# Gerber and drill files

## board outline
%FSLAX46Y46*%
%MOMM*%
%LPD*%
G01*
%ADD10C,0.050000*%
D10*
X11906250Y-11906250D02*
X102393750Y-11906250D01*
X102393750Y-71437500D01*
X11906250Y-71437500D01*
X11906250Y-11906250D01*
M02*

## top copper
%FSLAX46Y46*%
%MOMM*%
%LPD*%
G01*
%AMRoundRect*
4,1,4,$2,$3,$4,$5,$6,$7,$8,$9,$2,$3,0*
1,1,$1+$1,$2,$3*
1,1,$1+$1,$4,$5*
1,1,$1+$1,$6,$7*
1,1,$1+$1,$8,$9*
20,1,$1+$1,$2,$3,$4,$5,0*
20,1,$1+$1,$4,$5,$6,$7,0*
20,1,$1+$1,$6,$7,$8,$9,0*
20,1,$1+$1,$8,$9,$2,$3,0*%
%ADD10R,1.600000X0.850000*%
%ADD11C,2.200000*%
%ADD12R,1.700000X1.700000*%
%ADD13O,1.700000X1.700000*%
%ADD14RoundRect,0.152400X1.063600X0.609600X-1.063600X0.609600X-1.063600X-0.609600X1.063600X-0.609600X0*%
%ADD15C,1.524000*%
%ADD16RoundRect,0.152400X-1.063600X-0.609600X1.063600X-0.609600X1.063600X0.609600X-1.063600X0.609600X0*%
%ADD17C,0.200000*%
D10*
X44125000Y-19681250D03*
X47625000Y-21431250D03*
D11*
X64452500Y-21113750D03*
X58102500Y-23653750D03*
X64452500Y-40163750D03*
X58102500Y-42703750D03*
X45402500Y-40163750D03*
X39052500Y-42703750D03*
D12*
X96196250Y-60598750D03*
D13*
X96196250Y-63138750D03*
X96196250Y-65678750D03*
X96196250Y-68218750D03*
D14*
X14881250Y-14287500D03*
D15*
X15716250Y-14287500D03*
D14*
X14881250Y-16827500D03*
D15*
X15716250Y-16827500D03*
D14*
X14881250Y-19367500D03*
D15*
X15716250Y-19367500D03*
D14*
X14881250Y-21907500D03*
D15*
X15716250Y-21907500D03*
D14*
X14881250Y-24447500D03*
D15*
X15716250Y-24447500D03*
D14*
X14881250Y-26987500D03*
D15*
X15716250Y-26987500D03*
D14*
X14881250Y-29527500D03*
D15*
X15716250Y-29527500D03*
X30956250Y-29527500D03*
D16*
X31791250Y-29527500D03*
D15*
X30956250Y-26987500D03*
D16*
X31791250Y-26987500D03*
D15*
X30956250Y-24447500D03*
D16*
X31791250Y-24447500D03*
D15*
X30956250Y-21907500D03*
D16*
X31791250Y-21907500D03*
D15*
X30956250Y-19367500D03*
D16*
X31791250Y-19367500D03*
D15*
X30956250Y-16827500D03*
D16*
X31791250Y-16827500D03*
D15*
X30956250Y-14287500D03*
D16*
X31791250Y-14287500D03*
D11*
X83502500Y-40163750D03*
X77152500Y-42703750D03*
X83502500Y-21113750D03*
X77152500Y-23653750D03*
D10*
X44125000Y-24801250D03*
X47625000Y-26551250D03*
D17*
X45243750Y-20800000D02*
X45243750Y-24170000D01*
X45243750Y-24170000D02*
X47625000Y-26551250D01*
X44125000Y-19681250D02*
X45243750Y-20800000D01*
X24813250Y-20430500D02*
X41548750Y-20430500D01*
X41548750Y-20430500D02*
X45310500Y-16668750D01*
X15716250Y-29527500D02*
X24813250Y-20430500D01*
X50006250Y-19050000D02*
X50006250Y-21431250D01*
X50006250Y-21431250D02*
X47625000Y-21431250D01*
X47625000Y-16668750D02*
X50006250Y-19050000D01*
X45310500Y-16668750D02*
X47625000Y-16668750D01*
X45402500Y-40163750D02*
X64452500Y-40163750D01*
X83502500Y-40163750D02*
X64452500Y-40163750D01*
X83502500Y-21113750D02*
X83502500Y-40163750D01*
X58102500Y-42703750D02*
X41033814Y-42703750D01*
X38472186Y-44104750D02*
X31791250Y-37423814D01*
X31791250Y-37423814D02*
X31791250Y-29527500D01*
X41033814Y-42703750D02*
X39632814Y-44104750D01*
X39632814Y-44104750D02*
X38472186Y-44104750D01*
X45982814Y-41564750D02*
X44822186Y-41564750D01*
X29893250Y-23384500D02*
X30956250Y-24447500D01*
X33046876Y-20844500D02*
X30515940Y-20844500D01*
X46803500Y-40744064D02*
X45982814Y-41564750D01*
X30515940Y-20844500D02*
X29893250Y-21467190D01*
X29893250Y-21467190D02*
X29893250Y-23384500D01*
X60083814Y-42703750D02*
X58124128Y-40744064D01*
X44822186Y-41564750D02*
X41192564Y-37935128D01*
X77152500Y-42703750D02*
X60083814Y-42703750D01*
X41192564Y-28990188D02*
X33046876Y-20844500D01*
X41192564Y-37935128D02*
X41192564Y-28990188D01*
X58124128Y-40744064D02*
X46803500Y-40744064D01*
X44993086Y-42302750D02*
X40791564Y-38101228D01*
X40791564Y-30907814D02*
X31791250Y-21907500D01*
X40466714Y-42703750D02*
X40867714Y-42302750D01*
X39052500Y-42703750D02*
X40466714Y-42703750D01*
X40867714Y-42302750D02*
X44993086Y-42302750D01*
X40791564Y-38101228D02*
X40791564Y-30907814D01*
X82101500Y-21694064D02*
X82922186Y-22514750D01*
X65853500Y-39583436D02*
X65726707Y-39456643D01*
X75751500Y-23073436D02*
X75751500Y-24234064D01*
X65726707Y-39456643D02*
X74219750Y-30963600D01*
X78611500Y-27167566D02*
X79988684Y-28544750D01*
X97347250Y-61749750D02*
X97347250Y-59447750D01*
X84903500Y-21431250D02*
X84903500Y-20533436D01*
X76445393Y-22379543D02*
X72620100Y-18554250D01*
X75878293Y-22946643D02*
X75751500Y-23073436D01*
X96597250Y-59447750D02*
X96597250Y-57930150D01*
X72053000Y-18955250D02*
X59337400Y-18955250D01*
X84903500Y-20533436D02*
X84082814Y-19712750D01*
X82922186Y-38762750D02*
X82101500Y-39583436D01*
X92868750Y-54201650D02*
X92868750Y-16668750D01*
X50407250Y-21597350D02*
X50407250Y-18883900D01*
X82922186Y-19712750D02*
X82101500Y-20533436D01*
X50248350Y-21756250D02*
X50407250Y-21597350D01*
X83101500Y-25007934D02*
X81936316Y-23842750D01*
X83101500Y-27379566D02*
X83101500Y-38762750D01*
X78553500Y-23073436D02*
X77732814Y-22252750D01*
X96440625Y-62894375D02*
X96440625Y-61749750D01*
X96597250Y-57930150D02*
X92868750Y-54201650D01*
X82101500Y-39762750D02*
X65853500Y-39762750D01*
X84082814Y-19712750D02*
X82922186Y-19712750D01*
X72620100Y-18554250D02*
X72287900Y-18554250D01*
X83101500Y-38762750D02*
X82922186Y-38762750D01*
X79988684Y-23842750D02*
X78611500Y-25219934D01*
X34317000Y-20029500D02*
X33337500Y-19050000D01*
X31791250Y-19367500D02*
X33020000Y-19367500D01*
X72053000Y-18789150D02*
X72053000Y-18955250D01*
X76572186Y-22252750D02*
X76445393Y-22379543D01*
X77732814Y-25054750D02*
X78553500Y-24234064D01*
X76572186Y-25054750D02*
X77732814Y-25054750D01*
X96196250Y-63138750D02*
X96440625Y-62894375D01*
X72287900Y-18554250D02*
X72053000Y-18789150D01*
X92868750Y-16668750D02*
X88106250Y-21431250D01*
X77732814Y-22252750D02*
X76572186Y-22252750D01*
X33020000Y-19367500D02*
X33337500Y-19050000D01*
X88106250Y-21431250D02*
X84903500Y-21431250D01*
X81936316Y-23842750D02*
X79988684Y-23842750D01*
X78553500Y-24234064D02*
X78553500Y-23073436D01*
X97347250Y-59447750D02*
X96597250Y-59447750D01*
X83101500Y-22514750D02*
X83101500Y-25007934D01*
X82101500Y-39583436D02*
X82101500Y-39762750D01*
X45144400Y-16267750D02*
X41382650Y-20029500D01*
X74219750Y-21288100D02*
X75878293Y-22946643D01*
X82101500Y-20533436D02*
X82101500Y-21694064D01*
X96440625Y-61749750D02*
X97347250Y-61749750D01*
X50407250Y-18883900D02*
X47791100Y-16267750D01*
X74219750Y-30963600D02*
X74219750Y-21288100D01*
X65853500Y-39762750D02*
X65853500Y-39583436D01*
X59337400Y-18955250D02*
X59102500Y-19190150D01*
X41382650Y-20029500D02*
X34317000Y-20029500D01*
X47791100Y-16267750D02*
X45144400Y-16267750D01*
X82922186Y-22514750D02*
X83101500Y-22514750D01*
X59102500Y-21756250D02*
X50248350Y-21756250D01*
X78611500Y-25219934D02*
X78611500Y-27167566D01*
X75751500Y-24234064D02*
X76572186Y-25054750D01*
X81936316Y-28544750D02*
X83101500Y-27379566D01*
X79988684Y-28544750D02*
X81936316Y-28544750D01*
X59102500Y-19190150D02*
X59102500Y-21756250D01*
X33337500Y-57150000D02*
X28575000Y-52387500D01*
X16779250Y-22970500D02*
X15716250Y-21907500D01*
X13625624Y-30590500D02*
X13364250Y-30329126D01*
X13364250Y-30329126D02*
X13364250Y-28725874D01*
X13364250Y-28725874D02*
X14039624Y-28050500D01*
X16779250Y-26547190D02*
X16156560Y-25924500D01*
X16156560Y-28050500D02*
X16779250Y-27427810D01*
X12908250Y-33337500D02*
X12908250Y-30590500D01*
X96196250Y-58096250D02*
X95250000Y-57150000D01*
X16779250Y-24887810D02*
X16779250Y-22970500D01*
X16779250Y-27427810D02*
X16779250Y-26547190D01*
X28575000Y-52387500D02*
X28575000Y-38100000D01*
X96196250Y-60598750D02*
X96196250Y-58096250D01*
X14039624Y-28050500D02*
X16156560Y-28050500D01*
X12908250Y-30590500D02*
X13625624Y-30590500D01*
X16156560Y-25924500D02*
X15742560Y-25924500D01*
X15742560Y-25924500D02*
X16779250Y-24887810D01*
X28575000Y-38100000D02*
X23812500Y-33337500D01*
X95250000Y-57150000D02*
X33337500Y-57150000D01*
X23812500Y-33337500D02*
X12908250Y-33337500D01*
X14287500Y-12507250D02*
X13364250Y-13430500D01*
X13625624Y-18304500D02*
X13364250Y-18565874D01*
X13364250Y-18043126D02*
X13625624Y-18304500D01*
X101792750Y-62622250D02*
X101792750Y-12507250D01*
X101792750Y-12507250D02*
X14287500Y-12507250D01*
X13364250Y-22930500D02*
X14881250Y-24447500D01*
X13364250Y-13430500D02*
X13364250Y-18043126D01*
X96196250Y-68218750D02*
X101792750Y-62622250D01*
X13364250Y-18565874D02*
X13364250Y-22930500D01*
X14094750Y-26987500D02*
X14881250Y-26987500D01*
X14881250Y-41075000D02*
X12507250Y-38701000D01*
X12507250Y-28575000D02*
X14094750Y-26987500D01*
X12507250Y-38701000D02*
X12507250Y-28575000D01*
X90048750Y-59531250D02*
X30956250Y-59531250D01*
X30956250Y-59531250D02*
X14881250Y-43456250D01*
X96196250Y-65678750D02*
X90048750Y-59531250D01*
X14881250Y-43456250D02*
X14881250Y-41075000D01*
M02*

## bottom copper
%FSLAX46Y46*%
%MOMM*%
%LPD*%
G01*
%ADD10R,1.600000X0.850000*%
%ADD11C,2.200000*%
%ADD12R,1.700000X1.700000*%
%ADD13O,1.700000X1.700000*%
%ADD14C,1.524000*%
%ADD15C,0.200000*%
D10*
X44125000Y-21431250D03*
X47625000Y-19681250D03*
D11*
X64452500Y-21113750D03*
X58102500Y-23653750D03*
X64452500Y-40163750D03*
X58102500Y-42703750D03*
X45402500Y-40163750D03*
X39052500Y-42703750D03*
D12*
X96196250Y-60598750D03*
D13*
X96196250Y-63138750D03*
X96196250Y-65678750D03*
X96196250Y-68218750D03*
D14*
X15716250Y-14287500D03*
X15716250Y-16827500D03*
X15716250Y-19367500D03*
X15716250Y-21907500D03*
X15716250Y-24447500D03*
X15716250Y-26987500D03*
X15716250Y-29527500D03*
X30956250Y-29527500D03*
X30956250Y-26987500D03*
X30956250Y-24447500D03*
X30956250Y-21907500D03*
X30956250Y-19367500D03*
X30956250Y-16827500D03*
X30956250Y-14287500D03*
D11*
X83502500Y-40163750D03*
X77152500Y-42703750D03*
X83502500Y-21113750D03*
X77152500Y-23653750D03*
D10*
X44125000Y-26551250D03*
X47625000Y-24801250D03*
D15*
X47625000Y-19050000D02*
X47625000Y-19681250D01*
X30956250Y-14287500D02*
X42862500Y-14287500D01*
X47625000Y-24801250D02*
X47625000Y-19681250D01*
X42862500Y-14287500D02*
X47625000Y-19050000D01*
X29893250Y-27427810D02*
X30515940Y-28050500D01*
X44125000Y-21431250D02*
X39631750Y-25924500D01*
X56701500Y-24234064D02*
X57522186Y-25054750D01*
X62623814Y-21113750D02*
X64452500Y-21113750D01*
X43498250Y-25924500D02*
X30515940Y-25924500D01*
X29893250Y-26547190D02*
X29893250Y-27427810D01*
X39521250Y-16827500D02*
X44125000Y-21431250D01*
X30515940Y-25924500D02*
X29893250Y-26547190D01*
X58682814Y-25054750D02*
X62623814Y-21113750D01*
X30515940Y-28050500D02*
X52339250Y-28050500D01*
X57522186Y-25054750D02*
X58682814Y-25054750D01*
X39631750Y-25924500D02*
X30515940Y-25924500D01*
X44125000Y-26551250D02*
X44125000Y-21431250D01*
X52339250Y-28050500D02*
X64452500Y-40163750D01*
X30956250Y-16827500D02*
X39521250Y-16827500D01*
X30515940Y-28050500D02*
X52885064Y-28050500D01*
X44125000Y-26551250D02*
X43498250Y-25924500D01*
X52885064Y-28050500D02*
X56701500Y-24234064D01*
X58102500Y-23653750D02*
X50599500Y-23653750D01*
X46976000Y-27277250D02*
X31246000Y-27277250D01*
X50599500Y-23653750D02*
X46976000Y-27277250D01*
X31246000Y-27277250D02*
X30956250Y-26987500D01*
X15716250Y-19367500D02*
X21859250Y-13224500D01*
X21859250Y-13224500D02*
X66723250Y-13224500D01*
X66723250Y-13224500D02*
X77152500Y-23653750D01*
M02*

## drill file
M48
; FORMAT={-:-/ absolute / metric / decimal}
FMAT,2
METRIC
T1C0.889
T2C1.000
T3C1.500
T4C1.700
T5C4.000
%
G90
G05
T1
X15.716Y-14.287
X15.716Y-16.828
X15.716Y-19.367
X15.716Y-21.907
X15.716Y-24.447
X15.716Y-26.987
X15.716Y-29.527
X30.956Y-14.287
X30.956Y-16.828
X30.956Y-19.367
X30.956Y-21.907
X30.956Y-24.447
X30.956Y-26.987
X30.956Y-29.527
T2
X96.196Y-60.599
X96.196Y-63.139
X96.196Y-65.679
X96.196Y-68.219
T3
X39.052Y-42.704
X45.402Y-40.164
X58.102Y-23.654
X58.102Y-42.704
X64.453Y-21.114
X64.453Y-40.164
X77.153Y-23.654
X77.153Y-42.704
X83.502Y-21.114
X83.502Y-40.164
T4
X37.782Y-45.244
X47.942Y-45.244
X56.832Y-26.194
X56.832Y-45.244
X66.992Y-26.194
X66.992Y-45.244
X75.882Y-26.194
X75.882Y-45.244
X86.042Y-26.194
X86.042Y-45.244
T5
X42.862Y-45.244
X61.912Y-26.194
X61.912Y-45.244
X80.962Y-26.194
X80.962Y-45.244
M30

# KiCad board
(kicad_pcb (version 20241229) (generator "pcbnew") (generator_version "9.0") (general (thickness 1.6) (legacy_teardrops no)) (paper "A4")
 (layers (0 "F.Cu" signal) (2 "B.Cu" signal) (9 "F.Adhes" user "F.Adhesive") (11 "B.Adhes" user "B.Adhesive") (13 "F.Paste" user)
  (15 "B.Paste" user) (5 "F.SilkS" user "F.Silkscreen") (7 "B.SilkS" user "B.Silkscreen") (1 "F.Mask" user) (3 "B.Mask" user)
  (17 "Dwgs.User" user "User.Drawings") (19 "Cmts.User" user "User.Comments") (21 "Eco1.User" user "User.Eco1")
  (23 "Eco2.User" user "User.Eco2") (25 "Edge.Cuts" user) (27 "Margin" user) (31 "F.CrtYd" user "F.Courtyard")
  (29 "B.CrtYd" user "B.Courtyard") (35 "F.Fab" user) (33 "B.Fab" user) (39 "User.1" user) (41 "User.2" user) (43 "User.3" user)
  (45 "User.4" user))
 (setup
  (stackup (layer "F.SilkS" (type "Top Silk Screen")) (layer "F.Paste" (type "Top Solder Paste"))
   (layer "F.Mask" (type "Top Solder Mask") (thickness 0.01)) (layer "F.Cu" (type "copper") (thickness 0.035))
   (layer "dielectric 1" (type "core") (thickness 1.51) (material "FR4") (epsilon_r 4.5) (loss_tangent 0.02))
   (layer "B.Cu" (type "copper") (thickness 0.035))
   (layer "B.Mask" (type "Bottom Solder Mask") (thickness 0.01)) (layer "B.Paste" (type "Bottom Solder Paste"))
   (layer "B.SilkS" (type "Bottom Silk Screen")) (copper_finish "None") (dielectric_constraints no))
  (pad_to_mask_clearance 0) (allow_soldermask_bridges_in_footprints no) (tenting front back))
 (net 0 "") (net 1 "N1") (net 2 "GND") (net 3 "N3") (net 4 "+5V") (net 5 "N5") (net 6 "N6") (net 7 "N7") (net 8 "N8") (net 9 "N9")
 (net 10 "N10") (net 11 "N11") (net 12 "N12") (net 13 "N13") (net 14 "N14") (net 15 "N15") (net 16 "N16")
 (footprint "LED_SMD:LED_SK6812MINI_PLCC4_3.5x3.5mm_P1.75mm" (layer "F.Cu") (at 45.875 20.55625)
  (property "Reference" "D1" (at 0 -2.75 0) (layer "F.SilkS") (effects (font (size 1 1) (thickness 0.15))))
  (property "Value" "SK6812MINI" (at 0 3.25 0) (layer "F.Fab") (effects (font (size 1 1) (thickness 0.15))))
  (pad "1" smd rect (at -1.75 -0.875) (size 1.6 0.85) (layers "F.Cu" "F.Mask" "F.Paste") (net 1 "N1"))
  (pad "2" smd rect (at -1.75 0.875) (size 1.6 0.85) (layers "F.Mask" "B.Cu" "F.Paste") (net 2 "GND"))
  (pad "3" smd rect (at 1.75 0.875) (size 1.6 0.85) (layers "F.Cu" "F.Mask" "F.Paste") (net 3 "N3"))
  (pad "4" smd rect (at 1.75 -0.875) (size 1.6 0.85) (layers "F.Mask" "B.Cu" "F.Paste") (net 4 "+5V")))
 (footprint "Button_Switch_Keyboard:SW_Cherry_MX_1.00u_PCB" (layer "F.Cu") (at 64.4525 21.11375)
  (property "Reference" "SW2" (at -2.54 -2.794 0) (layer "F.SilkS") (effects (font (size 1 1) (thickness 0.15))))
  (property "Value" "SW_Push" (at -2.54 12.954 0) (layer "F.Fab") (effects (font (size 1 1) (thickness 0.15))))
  (pad "" np_thru_hole circle (at -7.62 5.08) (size 1.7 1.7) (drill 1.7) (layers "*.Cu" "*.Mask"))
  (pad "" np_thru_hole circle (at -2.54 5.08) (size 4 4) (drill 4) (layers "*.Cu" "*.Mask"))
  (pad "" np_thru_hole circle (at 2.54 5.08) (size 1.7 1.7) (drill 1.7) (layers "*.Cu" "*.Mask"))
  (pad "1" thru_hole circle (at 0 0) (size 2.2 2.2) (drill 1.5) (layers "*.Cu" "*.Mask") (remove_unused_layers no) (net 2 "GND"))
  (pad "2" thru_hole circle (at -6.35 2.54) (size 2.2 2.2) (drill 1.5) (layers "*.Cu" "*.Mask") (remove_unused_layers no) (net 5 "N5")))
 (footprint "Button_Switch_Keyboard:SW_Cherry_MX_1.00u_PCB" (layer "F.Cu") (at 64.4525 40.16375)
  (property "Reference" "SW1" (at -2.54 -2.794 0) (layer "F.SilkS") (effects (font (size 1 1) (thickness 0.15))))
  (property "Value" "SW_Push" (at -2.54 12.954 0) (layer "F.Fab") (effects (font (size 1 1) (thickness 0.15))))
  (pad "" np_thru_hole circle (at -7.62 5.08) (size 1.7 1.7) (drill 1.7) (layers "*.Cu" "*.Mask"))
  (pad "" np_thru_hole circle (at -2.54 5.08) (size 4 4) (drill 4) (layers "*.Cu" "*.Mask"))
  (pad "" np_thru_hole circle (at 2.54 5.08) (size 1.7 1.7) (drill 1.7) (layers "*.Cu" "*.Mask"))
  (pad "1" thru_hole circle (at 0 0) (size 2.2 2.2) (drill 1.5) (layers "*.Cu" "*.Mask") (remove_unused_layers no) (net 2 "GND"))
  (pad "2" thru_hole circle (at -6.35 2.54) (size 2.2 2.2) (drill 1.5) (layers "*.Cu" "*.Mask") (remove_unused_layers no) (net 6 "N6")))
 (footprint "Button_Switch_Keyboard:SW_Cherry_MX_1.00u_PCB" (layer "F.Cu") (at 45.4025 40.16375)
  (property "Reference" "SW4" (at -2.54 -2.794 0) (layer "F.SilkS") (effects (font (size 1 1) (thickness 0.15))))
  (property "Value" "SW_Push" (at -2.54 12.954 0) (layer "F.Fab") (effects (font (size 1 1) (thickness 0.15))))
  (pad "" np_thru_hole circle (at -7.62 5.08) (size 1.7 1.7) (drill 1.7) (layers "*.Cu" "*.Mask"))
  (pad "" np_thru_hole circle (at -2.54 5.08) (size 4 4) (drill 4) (layers "*.Cu" "*.Mask"))
  (pad "" np_thru_hole circle (at 2.54 5.08) (size 1.7 1.7) (drill 1.7) (layers "*.Cu" "*.Mask"))
  (pad "1" thru_hole circle (at 0 0) (size 2.2 2.2) (drill 1.5) (layers "*.Cu" "*.Mask") (remove_unused_layers no) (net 2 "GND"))
  (pad "2" thru_hole circle (at -6.35 2.54) (size 2.2 2.2) (drill 1.5) (layers "*.Cu" "*.Mask") (remove_unused_layers no) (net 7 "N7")))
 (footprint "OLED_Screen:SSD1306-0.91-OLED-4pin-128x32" (layer "F.Cu") (at 59.69625 58.40875)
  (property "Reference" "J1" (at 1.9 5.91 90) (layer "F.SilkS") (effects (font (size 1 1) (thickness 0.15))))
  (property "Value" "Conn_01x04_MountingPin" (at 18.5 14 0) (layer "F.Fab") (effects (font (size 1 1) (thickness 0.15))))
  (pad "1" thru_hole rect (at 36.5 2.19) (size 1.7 1.7) (drill 1) (layers "*.Cu" "*.Mask") (remove_unused_layers no) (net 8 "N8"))
  (pad "2" thru_hole oval (at 36.5 4.73) (size 1.7 1.7) (drill 1) (layers "*.Cu" "*.Mask") (remove_unused_layers no) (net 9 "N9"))
  (pad "3" thru_hole oval (at 36.5 7.27) (size 1.7 1.7) (drill 1) (layers "*.Cu" "*.Mask") (remove_unused_layers no) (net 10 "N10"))
  (pad "4" thru_hole oval (at 36.5 9.81) (size 1.7 1.7) (drill 1) (layers "*.Cu" "*.Mask") (remove_unused_layers no) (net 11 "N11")))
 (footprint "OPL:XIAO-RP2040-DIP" (layer "F.Cu") (at 23.33625 21.9075)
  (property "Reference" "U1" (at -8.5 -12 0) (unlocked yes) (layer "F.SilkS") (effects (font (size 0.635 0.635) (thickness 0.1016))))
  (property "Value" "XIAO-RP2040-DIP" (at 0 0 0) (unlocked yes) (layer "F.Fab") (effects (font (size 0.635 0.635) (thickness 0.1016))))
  (pad "1" smd roundrect (at -8.455 -7.62 180) (size 2.432 1.524) (layers "F.Cu" "F.Mask") (roundrect_rratio 0.1) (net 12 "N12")
   (thermal_bridge_angle 45))
  (pad "1" thru_hole circle (at -7.62 -7.62 180) (size 1.524 1.524) (drill 0.889) (layers "*.Cu" "*.Mask") (remove_unused_layers no)
   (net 12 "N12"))
  (pad "2" smd roundrect (at -8.455 -5.08 180) (size 2.432 1.524) (layers "F.Cu" "F.Mask") (roundrect_rratio 0.1) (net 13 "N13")
   (thermal_bridge_angle 45))
  (pad "2" thru_hole circle (at -7.62 -5.08 180) (size 1.524 1.524) (drill 0.889) (layers "*.Cu" "*.Mask") (remove_unused_layers no)
   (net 13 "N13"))
  (pad "3" smd roundrect (at -8.455 -2.54 180) (size 2.432 1.524) (layers "F.Cu" "F.Mask") (roundrect_rratio 0.1) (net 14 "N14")
   (thermal_bridge_angle 45))
  (pad "3" thru_hole circle (at -7.62 -2.54 180) (size 1.524 1.524) (drill 0.889) (layers "*.Cu" "*.Mask") (remove_unused_layers no)
   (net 14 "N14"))
  (pad "4" smd roundrect (at -8.455 0 180) (size 2.432 1.524) (layers "F.Cu" "F.Mask") (roundrect_rratio 0.1) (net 8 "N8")
   (thermal_bridge_angle 45))
  (pad "4" thru_hole circle (at -7.62 0 180) (size 1.524 1.524) (drill 0.889) (layers "*.Cu" "*.Mask") (remove_unused_layers no)
   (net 8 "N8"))
  (pad "5" smd roundrect (at -8.455 2.54 180) (size 2.432 1.524) (layers "F.Cu" "F.Mask") (roundrect_rratio 0.1) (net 11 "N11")
   (thermal_bridge_angle 45))
  (pad "5" thru_hole circle (at -7.62 2.54 180) (size 1.524 1.524) (drill 0.889) (layers "*.Cu" "*.Mask") (remove_unused_layers no)
   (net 11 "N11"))
  (pad "6" smd roundrect (at -8.455 5.08 180) (size 2.432 1.524) (layers "F.Cu" "F.Mask") (roundrect_rratio 0.1) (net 10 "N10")
   (thermal_bridge_angle 45))
  (pad "6" thru_hole circle (at -7.62 5.08 180) (size 1.524 1.524) (drill 0.889) (layers "*.Cu" "*.Mask") (remove_unused_layers no)
   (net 10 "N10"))
  (pad "7" smd roundrect (at -8.455 7.62 180) (size 2.432 1.524) (layers "F.Cu" "F.Mask") (roundrect_rratio 0.1) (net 3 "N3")
   (thermal_bridge_angle 45))
  (pad "7" thru_hole circle (at -7.62 7.62 180) (size 1.524 1.524) (drill 0.889) (layers "*.Cu" "*.Mask") (remove_unused_layers no)
   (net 3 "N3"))
  (pad "8" thru_hole circle (at 7.62 7.62) (size 1.524 1.524) (drill 0.889) (layers "*.Cu" "*.Mask") (remove_unused_layers no) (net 6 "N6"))
  (pad "8" smd roundrect (at 8.455 7.62) (size 2.432 1.524) (layers "F.Cu" "F.Mask") (roundrect_rratio 0.1) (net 6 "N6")
   (thermal_bridge_angle 45))
  (pad "9" thru_hole circle (at 7.62 5.08) (size 1.524 1.524) (drill 0.889) (layers "*.Cu" "*.Mask") (remove_unused_layers no) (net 5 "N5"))
  (pad "9" smd roundrect (at 8.455 5.08) (size 2.432 1.524) (layers "F.Cu" "F.Mask") (roundrect_rratio 0.1) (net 5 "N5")
   (thermal_bridge_angle 45))
  (pad "10" thru_hole circle (at 7.62 2.54) (size 1.524 1.524) (drill 0.889) (layers "*.Cu" "*.Mask") (remove_unused_layers no)
   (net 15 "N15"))
  (pad "10" smd roundrect (at 8.455 2.54) (size 2.432 1.524) (layers "F.Cu" "F.Mask") (roundrect_rratio 0.1) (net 15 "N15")
   (thermal_bridge_angle 45))
  (pad "11" thru_hole circle (at 7.62 0) (size 1.524 1.524) (drill 0.889) (layers "*.Cu" "*.Mask") (remove_unused_layers no) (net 7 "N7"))
  (pad "11" smd roundrect (at 8.455 0) (size 2.432 1.524) (layers "F.Cu" "F.Mask") (roundrect_rratio 0.1) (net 7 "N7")
   (thermal_bridge_angle 45))
  (pad "12" thru_hole circle (at 7.62 -2.54) (size 1.524 1.524) (drill 0.889) (layers "*.Cu" "*.Mask") (remove_unused_layers no)
   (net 9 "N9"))
  (pad "12" smd roundrect (at 8.455 -2.54) (size 2.432 1.524) (layers "F.Cu" "F.Mask") (roundrect_rratio 0.1) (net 9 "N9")
   (thermal_bridge_angle 45))
  (pad "13" thru_hole circle (at 7.62 -5.08) (size 1.524 1.524) (drill 0.889) (layers "*.Cu" "*.Mask") (remove_unused_layers no)
   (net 2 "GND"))
  (pad "13" smd roundrect (at 8.455 -5.08) (size 2.432 1.524) (layers "F.Cu" "F.Mask") (roundrect_rratio 0.1) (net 2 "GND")
   (thermal_bridge_angle 45))
  (pad "14" thru_hole circle (at 7.62 -7.62) (size 1.524 1.524) (drill 0.889) (layers "*.Cu" "*.Mask") (remove_unused_layers no)
   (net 4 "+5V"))
  (pad "14" smd roundrect (at 8.455 -7.62) (size 2.432 1.524) (layers "F.Cu" "F.Mask") (roundrect_rratio 0.1) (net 4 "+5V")
   (thermal_bridge_angle 45)))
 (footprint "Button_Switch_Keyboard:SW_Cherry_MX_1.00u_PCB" (layer "F.Cu") (at 83.5025 40.16375)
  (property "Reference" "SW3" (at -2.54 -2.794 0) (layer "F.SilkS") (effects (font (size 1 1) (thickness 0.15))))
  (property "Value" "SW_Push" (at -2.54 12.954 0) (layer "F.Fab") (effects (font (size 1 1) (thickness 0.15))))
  (pad "" np_thru_hole circle (at -7.62 5.08) (size 1.7 1.7) (drill 1.7) (layers "*.Cu" "*.Mask"))
  (pad "" np_thru_hole circle (at -2.54 5.08) (size 4 4) (drill 4) (layers "*.Cu" "*.Mask"))
  (pad "" np_thru_hole circle (at 2.54 5.08) (size 1.7 1.7) (drill 1.7) (layers "*.Cu" "*.Mask"))
  (pad "1" thru_hole circle (at 0 0) (size 2.2 2.2) (drill 1.5) (layers "*.Cu" "*.Mask") (remove_unused_layers no) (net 2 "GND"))
  (pad "2" thru_hole circle (at -6.35 2.54) (size 2.2 2.2) (drill 1.5) (layers "*.Cu" "*.Mask") (remove_unused_layers no) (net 15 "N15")))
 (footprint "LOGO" (layer "F.Cu") (at 21.43125 61.9125)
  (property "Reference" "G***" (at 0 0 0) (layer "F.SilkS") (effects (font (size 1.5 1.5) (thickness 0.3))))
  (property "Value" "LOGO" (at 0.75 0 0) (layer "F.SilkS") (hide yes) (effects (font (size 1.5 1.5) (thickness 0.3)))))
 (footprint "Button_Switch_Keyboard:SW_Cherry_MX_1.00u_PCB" (layer "F.Cu") (at 83.5025 21.11375)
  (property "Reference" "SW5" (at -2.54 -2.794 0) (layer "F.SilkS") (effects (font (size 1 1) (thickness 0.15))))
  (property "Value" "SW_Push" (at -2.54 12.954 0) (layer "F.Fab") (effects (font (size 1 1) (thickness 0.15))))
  (pad "" np_thru_hole circle (at -7.62 5.08) (size 1.7 1.7) (drill 1.7) (layers "*.Cu" "*.Mask"))
  (pad "" np_thru_hole circle (at -2.54 5.08) (size 4 4) (drill 4) (layers "*.Cu" "*.Mask"))
  (pad "" np_thru_hole circle (at 2.54 5.08) (size 1.7 1.7) (drill 1.7) (layers "*.Cu" "*.Mask"))
  (pad "1" thru_hole circle (at 0 0) (size 2.2 2.2) (drill 1.5) (layers "*.Cu" "*.Mask") (remove_unused_layers no) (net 2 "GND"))
  (pad "2" thru_hole circle (at -6.35 2.54) (size 2.2 2.2) (drill 1.5) (layers "*.Cu" "*.Mask") (remove_unused_layers no) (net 14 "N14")))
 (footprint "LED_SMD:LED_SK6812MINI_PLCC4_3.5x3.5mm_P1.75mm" (layer "F.Cu") (at 45.875 25.67625)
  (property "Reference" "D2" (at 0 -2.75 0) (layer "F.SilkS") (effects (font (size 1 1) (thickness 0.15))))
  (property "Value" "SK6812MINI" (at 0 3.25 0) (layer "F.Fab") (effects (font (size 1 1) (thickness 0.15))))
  (pad "1" smd rect (at -1.75 -0.875) (size 1.6 0.85) (layers "F.Cu" "F.Mask" "F.Paste") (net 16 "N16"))
  (pad "2" smd rect (at -1.75 0.875) (size 1.6 0.85) (layers "F.Mask" "B.Cu" "F.Paste") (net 2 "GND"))
  (pad "3" smd rect (at 1.75 0.875) (size 1.6 0.85) (layers "F.Cu" "F.Mask" "F.Paste") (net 1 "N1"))
  (pad "4" smd rect (at 1.75 -0.875) (size 1.6 0.85) (layers "F.Mask" "B.Cu" "F.Paste") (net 4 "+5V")))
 (gr_rect (start 11.90625 11.90625) (end 102.39375 71.4375) (stroke (width 0.05) (type default)) (fill no) (layer "Edge.Cuts"))
 (segment (start 45.24375 20.8) (end 45.24375 24.17) (width 0.2) (layer "F.Cu") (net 1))
 (segment (start 45.24375 24.17) (end 47.625 26.55125) (width 0.2) (layer "F.Cu") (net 1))
 (segment (start 44.125 19.68125) (end 45.24375 20.8) (width 0.2) (layer "F.Cu") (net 1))
 (segment (start 47.625 19.05) (end 47.625 19.68125) (width 0.2) (layer "B.Cu") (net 4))
 (segment (start 30.95625 14.2875) (end 42.8625 14.2875) (width 0.2) (layer "B.Cu") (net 4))
 (segment (start 47.625 24.80125) (end 47.625 19.68125) (width 0.2) (layer "B.Cu") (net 4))
 (segment (start 42.8625 14.2875) (end 47.625 19.05) (width 0.2) (layer "B.Cu") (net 4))
 (segment (start 24.81325 20.4305) (end 41.54875 20.4305) (width 0.2) (layer "F.Cu") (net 3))
 (segment (start 41.54875 20.4305) (end 45.3105 16.66875) (width 0.2) (layer "F.Cu") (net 3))
 (segment (start 15.71625 29.5275) (end 24.81325 20.4305) (width 0.2) (layer "F.Cu") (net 3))
 (segment (start 50.00625 19.05) (end 50.00625 21.43125) (width 0.2) (layer "F.Cu") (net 3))
 (segment (start 50.00625 21.43125) (end 47.625 21.43125) (width 0.2) (layer "F.Cu") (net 3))
 (segment (start 47.625 16.66875) (end 50.00625 19.05) (width 0.2) (layer "F.Cu") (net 3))
 (segment (start 45.3105 16.66875) (end 47.625 16.66875) (width 0.2) (layer "F.Cu") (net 3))
 (segment (start 45.4025 40.16375) (end 64.4525 40.16375) (width 0.2) (layer "F.Cu") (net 2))
 (segment (start 83.5025 40.16375) (end 64.4525 40.16375) (width 0.2) (layer "F.Cu") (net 2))
 (segment (start 83.5025 21.11375) (end 83.5025 40.16375) (width 0.2) (layer "F.Cu") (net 2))
 (segment (start 29.89325 27.42781) (end 30.51594 28.0505) (width 0.2) (layer "B.Cu") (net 2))
 (segment (start 44.125 21.43125) (end 39.63175 25.9245) (width 0.2) (layer "B.Cu") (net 2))
 (segment (start 56.7015 24.234064) (end 57.522186 25.05475) (width 0.2) (layer "B.Cu") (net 2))
 (segment (start 62.623814 21.11375) (end 64.4525 21.11375) (width 0.2) (layer "B.Cu") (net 2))
 (segment (start 43.49825 25.9245) (end 30.51594 25.9245) (width 0.2) (layer "B.Cu") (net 2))
 (segment (start 29.89325 26.54719) (end 29.89325 27.42781) (width 0.2) (layer "B.Cu") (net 2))
 (segment (start 39.52125 16.8275) (end 44.125 21.43125) (width 0.2) (layer "B.Cu") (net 2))
 (segment (start 30.51594 25.9245) (end 29.89325 26.54719) (width 0.2) (layer "B.Cu") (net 2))
 (segment (start 58.682814 25.05475) (end 62.623814 21.11375) (width 0.2) (layer "B.Cu") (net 2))
 (segment (start 30.51594 28.0505) (end 52.33925 28.0505) (width 0.2) (layer "B.Cu") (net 2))
 (segment (start 57.522186 25.05475) (end 58.682814 25.05475) (width 0.2) (layer "B.Cu") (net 2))
 (segment (start 39.63175 25.9245) (end 30.51594 25.9245) (width 0.2) (layer "B.Cu") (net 2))
 (segment (start 44.125 26.55125) (end 44.125 21.43125) (width 0.2) (layer "B.Cu") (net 2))
 (segment (start 52.33925 28.0505) (end 64.4525 40.16375) (width 0.2) (layer "B.Cu") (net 2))
 (segment (start 30.95625 16.8275) (end 39.52125 16.8275) (width 0.2) (layer "B.Cu") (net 2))
 (segment (start 30.51594 28.0505) (end 52.885064 28.0505) (width 0.2) (layer "B.Cu") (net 2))
 (segment (start 44.125 26.55125) (end 43.49825 25.9245) (width 0.2) (layer "B.Cu") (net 2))
 (segment (start 52.885064 28.0505) (end 56.7015 24.234064) (width 0.2) (layer "B.Cu") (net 2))
 (segment (start 58.1025 42.70375) (end 41.033814 42.70375) (width 0.2) (layer "F.Cu") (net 6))
 (segment (start 38.472186 44.10475) (end 31.79125 37.423814) (width 0.2) (layer "F.Cu") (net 6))
 (segment (start 31.79125 37.423814) (end 31.79125 29.5275) (width 0.2) (layer "F.Cu") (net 6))
 (segment (start 41.033814 42.70375) (end 39.632814 44.10475) (width 0.2) (layer "F.Cu") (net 6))
 (segment (start 39.632814 44.10475) (end 38.472186 44.10475) (width 0.2) (layer "F.Cu") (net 6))
 (segment (start 58.1025 23.65375) (end 50.5995 23.65375) (width 0.2) (layer "B.Cu") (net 5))
 (segment (start 46.976 27.27725) (end 31.246 27.27725) (width 0.2) (layer "B.Cu") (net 5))
 (segment (start 50.5995 23.65375) (end 46.976 27.27725) (width 0.2) (layer "B.Cu") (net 5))
 (segment (start 31.246 27.27725) (end 30.95625 26.9875) (width 0.2) (layer "B.Cu") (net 5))
 (segment (start 45.982814 41.56475) (end 44.822186 41.56475) (width 0.2) (layer "F.Cu") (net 15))
 (segment (start 29.89325 23.3845) (end 30.95625 24.4475) (width 0.2) (layer "F.Cu") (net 15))
 (segment (start 33.046876 20.8445) (end 30.51594 20.8445) (width 0.2) (layer "F.Cu") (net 15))
 (segment (start 46.8035 40.744064) (end 45.982814 41.56475) (width 0.2) (layer "F.Cu") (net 15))
 (segment (start 30.51594 20.8445) (end 29.89325 21.46719) (width 0.2) (layer "F.Cu") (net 15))
 (segment (start 29.89325 21.46719) (end 29.89325 23.3845) (width 0.2) (layer "F.Cu") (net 15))
 (segment (start 60.083814 42.70375) (end 58.124128 40.744064) (width 0.2) (layer "F.Cu") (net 15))
 (segment (start 44.822186 41.56475) (end 41.192564 37.935128) (width 0.2) (layer "F.Cu") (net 15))
 (segment (start 77.1525 42.70375) (end 60.083814 42.70375) (width 0.2) (layer "F.Cu") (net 15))
 (segment (start 41.192564 28.990188) (end 33.046876 20.8445) (width 0.2) (layer "F.Cu") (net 15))
 (segment (start 41.192564 37.935128) (end 41.192564 28.990188) (width 0.2) (layer "F.Cu") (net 15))
 (segment (start 58.124128 40.744064) (end 46.8035 40.744064) (width 0.2) (layer "F.Cu") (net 15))
 (segment (start 44.993086 42.30275) (end 40.791564 38.101228) (width 0.2) (layer "F.Cu") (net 7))
 (segment (start 40.791564 30.907814) (end 31.79125 21.9075) (width 0.2) (layer "F.Cu") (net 7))
 (segment (start 40.466714 42.70375) (end 40.867714 42.30275) (width 0.2) (layer "F.Cu") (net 7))
 (segment (start 39.0525 42.70375) (end 40.466714 42.70375) (width 0.2) (layer "F.Cu") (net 7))
 (segment (start 40.867714 42.30275) (end 44.993086 42.30275) (width 0.2) (layer "F.Cu") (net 7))
 (segment (start 40.791564 38.101228) (end 40.791564 30.907814) (width 0.2) (layer "F.Cu") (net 7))
 (segment (start 82.1015 21.694064) (end 82.922186 22.51475) (width 0.2) (layer "F.Cu") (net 9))
 (segment (start 65.8535 39.583436) (end 65.726707 39.456643) (width 0.2) (layer "F.Cu") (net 9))
 (segment (start 75.7515 23.073436) (end 75.7515 24.234064) (width 0.2) (layer "F.Cu") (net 9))
 (segment (start 65.726707 39.456643) (end 74.21975 30.9636) (width 0.2) (layer "F.Cu") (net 9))
 (segment (start 78.6115 27.167566) (end 79.988684 28.54475) (width 0.2) (layer "F.Cu") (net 9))
 (segment (start 97.34725 61.74975) (end 97.34725 59.44775) (width 0.2) (layer "F.Cu") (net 9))
 (segment (start 84.9035 21.43125) (end 84.9035 20.533436) (width 0.2) (layer "F.Cu") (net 9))
 (segment (start 76.445393 22.379543) (end 72.6201 18.55425) (width 0.2) (layer "F.Cu") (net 9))
 (segment (start 75.878293 22.946643) (end 75.7515 23.073436) (width 0.2) (layer "F.Cu") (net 9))
 (segment (start 96.59725 59.44775) (end 96.59725 57.93015) (width 0.2) (layer "F.Cu") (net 9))
 (segment (start 72.053 18.95525) (end 59.3374 18.95525) (width 0.2) (layer "F.Cu") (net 9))
 (segment (start 84.9035 20.533436) (end 84.082814 19.71275) (width 0.2) (layer "F.Cu") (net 9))
 (segment (start 82.922186 38.76275) (end 82.1015 39.583436) (width 0.2) (layer "F.Cu") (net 9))
 (segment (start 92.86875 54.20165) (end 92.86875 16.66875) (width 0.2) (layer "F.Cu") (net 9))
 (segment (start 50.40725 21.59735) (end 50.40725 18.8839) (width 0.2) (layer "F.Cu") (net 9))
 (segment (start 82.922186 19.71275) (end 82.1015 20.533436) (width 0.2) (layer "F.Cu") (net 9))
 (segment (start 50.24835 21.75625) (end 50.40725 21.59735) (width 0.2) (layer "F.Cu") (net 9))
 (segment (start 83.1015 25.007934) (end 81.936316 23.84275) (width 0.2) (layer "F.Cu") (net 9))
 (segment (start 83.1015 27.379566) (end 83.1015 38.76275) (width 0.2) (layer "F.Cu") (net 9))
 (segment (start 78.5535 23.073436) (end 77.732814 22.25275) (width 0.2) (layer "F.Cu") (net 9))
 (segment (start 96.440625 62.894375) (end 96.440625 61.74975) (width 0.2) (layer "F.Cu") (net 9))
 (segment (start 96.59725 57.93015) (end 92.86875 54.20165) (width 0.2) (layer "F.Cu") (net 9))
 (segment (start 82.1015 39.76275) (end 65.8535 39.76275) (width 0.2) (layer "F.Cu") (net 9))
 (segment (start 84.082814 19.71275) (end 82.922186 19.71275) (width 0.2) (layer "F.Cu") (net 9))
 (segment (start 72.6201 18.55425) (end 72.2879 18.55425) (width 0.2) (layer "F.Cu") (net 9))
 (segment (start 83.1015 38.76275) (end 82.922186 38.76275) (width 0.2) (layer "F.Cu") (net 9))
 (segment (start 79.988684 23.84275) (end 78.6115 25.219934) (width 0.2) (layer "F.Cu") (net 9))
 (segment (start 34.317 20.0295) (end 33.3375 19.05) (width 0.2) (layer "F.Cu") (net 9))
 (segment (start 31.79125 19.3675) (end 33.02 19.3675) (width 0.2) (layer "F.Cu") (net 9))
 (segment (start 72.053 18.78915) (end 72.053 18.95525) (width 0.2) (layer "F.Cu") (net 9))
 (segment (start 76.572186 22.25275) (end 76.445393 22.379543) (width 0.2) (layer "F.Cu") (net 9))
 (segment (start 77.732814 25.05475) (end 78.5535 24.234064) (width 0.2) (layer "F.Cu") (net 9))
 (segment (start 76.572186 25.05475) (end 77.732814 25.05475) (width 0.2) (layer "F.Cu") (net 9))
 (segment (start 96.19625 63.13875) (end 96.440625 62.894375) (width 0.2) (layer "F.Cu") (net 9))
 (segment (start 72.2879 18.55425) (end 72.053 18.78915) (width 0.2) (layer "F.Cu") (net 9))
 (segment (start 92.86875 16.66875) (end 88.10625 21.43125) (width 0.2) (layer "F.Cu") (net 9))
 (segment (start 77.732814 22.25275) (end 76.572186 22.25275) (width 0.2) (layer "F.Cu") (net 9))
 (segment (start 33.02 19.3675) (end 33.3375 19.05) (width 0.2) (layer "F.Cu") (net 9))
 (segment (start 88.10625 21.43125) (end 84.9035 21.43125) (width 0.2) (layer "F.Cu") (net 9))
 (segment (start 81.936316 23.84275) (end 79.988684 23.84275) (width 0.2) (layer "F.Cu") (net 9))
 (segment (start 78.5535 24.234064) (end 78.5535 23.073436) (width 0.2) (layer "F.Cu") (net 9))
 (segment (start 97.34725 59.44775) (end 96.59725 59.44775) (width 0.2) (layer "F.Cu") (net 9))
 (segment (start 83.1015 22.51475) (end 83.1015 25.007934) (width 0.2) (layer "F.Cu") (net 9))
 (segment (start 82.1015 39.583436) (end 82.1015 39.76275) (width 0.2) (layer "F.Cu") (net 9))
 (segment (start 45.1444 16.26775) (end 41.38265 20.0295) (width 0.2) (layer "F.Cu") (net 9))
 (segment (start 74.21975 21.2881) (end 75.878293 22.946643) (width 0.2) (layer "F.Cu") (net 9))
 (segment (start 82.1015 20.533436) (end 82.1015 21.694064) (width 0.2) (layer "F.Cu") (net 9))
 (segment (start 96.440625 61.74975) (end 97.34725 61.74975) (width 0.2) (layer "F.Cu") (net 9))
 (segment (start 50.40725 18.8839) (end 47.7911 16.26775) (width 0.2) (layer "F.Cu") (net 9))
 (segment (start 74.21975 30.9636) (end 74.21975 21.2881) (width 0.2) (layer "F.Cu") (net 9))
 (segment (start 65.8535 39.76275) (end 65.8535 39.583436) (width 0.2) (layer "F.Cu") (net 9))
 (segment (start 59.3374 18.95525) (end 59.1025 19.19015) (width 0.2) (layer "F.Cu") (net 9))
 (segment (start 41.38265 20.0295) (end 34.317 20.0295) (width 0.2) (layer "F.Cu") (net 9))
 (segment (start 47.7911 16.26775) (end 45.1444 16.26775) (width 0.2) (layer "F.Cu") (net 9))
 (segment (start 82.922186 22.51475) (end 83.1015 22.51475) (width 0.2) (layer "F.Cu") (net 9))
 (segment (start 59.1025 21.75625) (end 50.24835 21.75625) (width 0.2) (layer "F.Cu") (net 9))
 (segment (start 78.6115 25.219934) (end 78.6115 27.167566) (width 0.2) (layer "F.Cu") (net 9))
 (segment (start 75.7515 24.234064) (end 76.572186 25.05475) (width 0.2) (layer "F.Cu") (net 9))
 (segment (start 81.936316 28.54475) (end 83.1015 27.379566) (width 0.2) (layer "F.Cu") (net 9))
 (segment (start 79.988684 28.54475) (end 81.936316 28.54475) (width 0.2) (layer "F.Cu") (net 9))
 (segment (start 59.1025 19.19015) (end 59.1025 21.75625) (width 0.2) (layer "F.Cu") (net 9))
 (segment (start 33.3375 57.15) (end 28.575 52.3875) (width 0.2) (layer "F.Cu") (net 8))
 (segment (start 16.77925 22.9705) (end 15.71625 21.9075) (width 0.2) (layer "F.Cu") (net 8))
 (segment (start 13.625624 30.5905) (end 13.36425 30.329126) (width 0.2) (layer "F.Cu") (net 8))
 (segment (start 13.36425 30.329126) (end 13.36425 28.725874) (width 0.2) (layer "F.Cu") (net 8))
 (segment (start 13.36425 28.725874) (end 14.039624 28.0505) (width 0.2) (layer "F.Cu") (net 8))
 (segment (start 16.77925 26.54719) (end 16.15656 25.9245) (width 0.2) (layer "F.Cu") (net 8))
 (segment (start 16.15656 28.0505) (end 16.77925 27.42781) (width 0.2) (layer "F.Cu") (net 8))
 (segment (start 12.90825 33.3375) (end 12.90825 30.5905) (width 0.2) (layer "F.Cu") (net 8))
 (segment (start 96.19625 58.09625) (end 95.25 57.15) (width 0.2) (layer "F.Cu") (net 8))
 (segment (start 16.77925 24.88781) (end 16.77925 22.9705) (width 0.2) (layer "F.Cu") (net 8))
 (segment (start 16.77925 27.42781) (end 16.77925 26.54719) (width 0.2) (layer "F.Cu") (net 8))
 (segment (start 28.575 52.3875) (end 28.575 38.1) (width 0.2) (layer "F.Cu") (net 8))
 (segment (start 96.19625 60.59875) (end 96.19625 58.09625) (width 0.2) (layer "F.Cu") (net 8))
 (segment (start 14.039624 28.0505) (end 16.15656 28.0505) (width 0.2) (layer "F.Cu") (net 8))
 (segment (start 12.90825 30.5905) (end 13.625624 30.5905) (width 0.2) (layer "F.Cu") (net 8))
 (segment (start 16.15656 25.9245) (end 15.74256 25.9245) (width 0.2) (layer "F.Cu") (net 8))
 (segment (start 15.74256 25.9245) (end 16.77925 24.88781) (width 0.2) (layer "F.Cu") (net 8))
 (segment (start 28.575 38.1) (end 23.8125 33.3375) (width 0.2) (layer "F.Cu") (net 8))
 (segment (start 95.25 57.15) (end 33.3375 57.15) (width 0.2) (layer "F.Cu") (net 8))
 (segment (start 23.8125 33.3375) (end 12.90825 33.3375) (width 0.2) (layer "F.Cu") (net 8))
 (segment (start 14.2875 12.50725) (end 13.36425 13.4305) (width 0.2) (layer "F.Cu") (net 11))
 (segment (start 13.625624 18.3045) (end 13.36425 18.565874) (width 0.2) (layer "F.Cu") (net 11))
 (segment (start 13.36425 18.043126) (end 13.625624 18.3045) (width 0.2) (layer "F.Cu") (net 11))
 (segment (start 101.79275 62.62225) (end 101.79275 12.50725) (width 0.2) (layer "F.Cu") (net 11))
 (segment (start 101.79275 12.50725) (end 14.2875 12.50725) (width 0.2) (layer "F.Cu") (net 11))
 (segment (start 13.36425 22.9305) (end 14.88125 24.4475) (width 0.2) (layer "F.Cu") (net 11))
 (segment (start 13.36425 13.4305) (end 13.36425 18.043126) (width 0.2) (layer "F.Cu") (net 11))
 (segment (start 96.19625 68.21875) (end 101.79275 62.62225) (width 0.2) (layer "F.Cu") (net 11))
 (segment (start 13.36425 18.565874) (end 13.36425 22.9305) (width 0.2) (layer "F.Cu") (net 11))
 (segment (start 14.09475 26.9875) (end 14.88125 26.9875) (width 0.2) (layer "F.Cu") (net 10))
 (segment (start 14.88125 41.075) (end 12.50725 38.701) (width 0.2) (layer "F.Cu") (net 10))
 (segment (start 12.50725 28.575) (end 14.09475 26.9875) (width 0.2) (layer "F.Cu") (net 10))
 (segment (start 12.50725 38.701) (end 12.50725 28.575) (width 0.2) (layer "F.Cu") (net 10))
 (segment (start 90.04875 59.53125) (end 30.95625 59.53125) (width 0.2) (layer "F.Cu") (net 10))
 (segment (start 30.95625 59.53125) (end 14.88125 43.45625) (width 0.2) (layer "F.Cu") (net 10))
 (segment (start 96.19625 65.67875) (end 90.04875 59.53125) (width 0.2) (layer "F.Cu") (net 10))
 (segment (start 14.88125 43.45625) (end 14.88125 41.075) (width 0.2) (layer "F.Cu") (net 10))
 (segment (start 15.71625 19.3675) (end 21.85925 13.2245) (width 0.2) (layer "B.Cu") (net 14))
 (segment (start 21.85925 13.2245) (end 66.72325 13.2245) (width 0.2) (layer "B.Cu") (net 14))
 (segment (start 66.72325 13.2245) (end 77.1525 23.65375) (width 0.2) (layer "B.Cu") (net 14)))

